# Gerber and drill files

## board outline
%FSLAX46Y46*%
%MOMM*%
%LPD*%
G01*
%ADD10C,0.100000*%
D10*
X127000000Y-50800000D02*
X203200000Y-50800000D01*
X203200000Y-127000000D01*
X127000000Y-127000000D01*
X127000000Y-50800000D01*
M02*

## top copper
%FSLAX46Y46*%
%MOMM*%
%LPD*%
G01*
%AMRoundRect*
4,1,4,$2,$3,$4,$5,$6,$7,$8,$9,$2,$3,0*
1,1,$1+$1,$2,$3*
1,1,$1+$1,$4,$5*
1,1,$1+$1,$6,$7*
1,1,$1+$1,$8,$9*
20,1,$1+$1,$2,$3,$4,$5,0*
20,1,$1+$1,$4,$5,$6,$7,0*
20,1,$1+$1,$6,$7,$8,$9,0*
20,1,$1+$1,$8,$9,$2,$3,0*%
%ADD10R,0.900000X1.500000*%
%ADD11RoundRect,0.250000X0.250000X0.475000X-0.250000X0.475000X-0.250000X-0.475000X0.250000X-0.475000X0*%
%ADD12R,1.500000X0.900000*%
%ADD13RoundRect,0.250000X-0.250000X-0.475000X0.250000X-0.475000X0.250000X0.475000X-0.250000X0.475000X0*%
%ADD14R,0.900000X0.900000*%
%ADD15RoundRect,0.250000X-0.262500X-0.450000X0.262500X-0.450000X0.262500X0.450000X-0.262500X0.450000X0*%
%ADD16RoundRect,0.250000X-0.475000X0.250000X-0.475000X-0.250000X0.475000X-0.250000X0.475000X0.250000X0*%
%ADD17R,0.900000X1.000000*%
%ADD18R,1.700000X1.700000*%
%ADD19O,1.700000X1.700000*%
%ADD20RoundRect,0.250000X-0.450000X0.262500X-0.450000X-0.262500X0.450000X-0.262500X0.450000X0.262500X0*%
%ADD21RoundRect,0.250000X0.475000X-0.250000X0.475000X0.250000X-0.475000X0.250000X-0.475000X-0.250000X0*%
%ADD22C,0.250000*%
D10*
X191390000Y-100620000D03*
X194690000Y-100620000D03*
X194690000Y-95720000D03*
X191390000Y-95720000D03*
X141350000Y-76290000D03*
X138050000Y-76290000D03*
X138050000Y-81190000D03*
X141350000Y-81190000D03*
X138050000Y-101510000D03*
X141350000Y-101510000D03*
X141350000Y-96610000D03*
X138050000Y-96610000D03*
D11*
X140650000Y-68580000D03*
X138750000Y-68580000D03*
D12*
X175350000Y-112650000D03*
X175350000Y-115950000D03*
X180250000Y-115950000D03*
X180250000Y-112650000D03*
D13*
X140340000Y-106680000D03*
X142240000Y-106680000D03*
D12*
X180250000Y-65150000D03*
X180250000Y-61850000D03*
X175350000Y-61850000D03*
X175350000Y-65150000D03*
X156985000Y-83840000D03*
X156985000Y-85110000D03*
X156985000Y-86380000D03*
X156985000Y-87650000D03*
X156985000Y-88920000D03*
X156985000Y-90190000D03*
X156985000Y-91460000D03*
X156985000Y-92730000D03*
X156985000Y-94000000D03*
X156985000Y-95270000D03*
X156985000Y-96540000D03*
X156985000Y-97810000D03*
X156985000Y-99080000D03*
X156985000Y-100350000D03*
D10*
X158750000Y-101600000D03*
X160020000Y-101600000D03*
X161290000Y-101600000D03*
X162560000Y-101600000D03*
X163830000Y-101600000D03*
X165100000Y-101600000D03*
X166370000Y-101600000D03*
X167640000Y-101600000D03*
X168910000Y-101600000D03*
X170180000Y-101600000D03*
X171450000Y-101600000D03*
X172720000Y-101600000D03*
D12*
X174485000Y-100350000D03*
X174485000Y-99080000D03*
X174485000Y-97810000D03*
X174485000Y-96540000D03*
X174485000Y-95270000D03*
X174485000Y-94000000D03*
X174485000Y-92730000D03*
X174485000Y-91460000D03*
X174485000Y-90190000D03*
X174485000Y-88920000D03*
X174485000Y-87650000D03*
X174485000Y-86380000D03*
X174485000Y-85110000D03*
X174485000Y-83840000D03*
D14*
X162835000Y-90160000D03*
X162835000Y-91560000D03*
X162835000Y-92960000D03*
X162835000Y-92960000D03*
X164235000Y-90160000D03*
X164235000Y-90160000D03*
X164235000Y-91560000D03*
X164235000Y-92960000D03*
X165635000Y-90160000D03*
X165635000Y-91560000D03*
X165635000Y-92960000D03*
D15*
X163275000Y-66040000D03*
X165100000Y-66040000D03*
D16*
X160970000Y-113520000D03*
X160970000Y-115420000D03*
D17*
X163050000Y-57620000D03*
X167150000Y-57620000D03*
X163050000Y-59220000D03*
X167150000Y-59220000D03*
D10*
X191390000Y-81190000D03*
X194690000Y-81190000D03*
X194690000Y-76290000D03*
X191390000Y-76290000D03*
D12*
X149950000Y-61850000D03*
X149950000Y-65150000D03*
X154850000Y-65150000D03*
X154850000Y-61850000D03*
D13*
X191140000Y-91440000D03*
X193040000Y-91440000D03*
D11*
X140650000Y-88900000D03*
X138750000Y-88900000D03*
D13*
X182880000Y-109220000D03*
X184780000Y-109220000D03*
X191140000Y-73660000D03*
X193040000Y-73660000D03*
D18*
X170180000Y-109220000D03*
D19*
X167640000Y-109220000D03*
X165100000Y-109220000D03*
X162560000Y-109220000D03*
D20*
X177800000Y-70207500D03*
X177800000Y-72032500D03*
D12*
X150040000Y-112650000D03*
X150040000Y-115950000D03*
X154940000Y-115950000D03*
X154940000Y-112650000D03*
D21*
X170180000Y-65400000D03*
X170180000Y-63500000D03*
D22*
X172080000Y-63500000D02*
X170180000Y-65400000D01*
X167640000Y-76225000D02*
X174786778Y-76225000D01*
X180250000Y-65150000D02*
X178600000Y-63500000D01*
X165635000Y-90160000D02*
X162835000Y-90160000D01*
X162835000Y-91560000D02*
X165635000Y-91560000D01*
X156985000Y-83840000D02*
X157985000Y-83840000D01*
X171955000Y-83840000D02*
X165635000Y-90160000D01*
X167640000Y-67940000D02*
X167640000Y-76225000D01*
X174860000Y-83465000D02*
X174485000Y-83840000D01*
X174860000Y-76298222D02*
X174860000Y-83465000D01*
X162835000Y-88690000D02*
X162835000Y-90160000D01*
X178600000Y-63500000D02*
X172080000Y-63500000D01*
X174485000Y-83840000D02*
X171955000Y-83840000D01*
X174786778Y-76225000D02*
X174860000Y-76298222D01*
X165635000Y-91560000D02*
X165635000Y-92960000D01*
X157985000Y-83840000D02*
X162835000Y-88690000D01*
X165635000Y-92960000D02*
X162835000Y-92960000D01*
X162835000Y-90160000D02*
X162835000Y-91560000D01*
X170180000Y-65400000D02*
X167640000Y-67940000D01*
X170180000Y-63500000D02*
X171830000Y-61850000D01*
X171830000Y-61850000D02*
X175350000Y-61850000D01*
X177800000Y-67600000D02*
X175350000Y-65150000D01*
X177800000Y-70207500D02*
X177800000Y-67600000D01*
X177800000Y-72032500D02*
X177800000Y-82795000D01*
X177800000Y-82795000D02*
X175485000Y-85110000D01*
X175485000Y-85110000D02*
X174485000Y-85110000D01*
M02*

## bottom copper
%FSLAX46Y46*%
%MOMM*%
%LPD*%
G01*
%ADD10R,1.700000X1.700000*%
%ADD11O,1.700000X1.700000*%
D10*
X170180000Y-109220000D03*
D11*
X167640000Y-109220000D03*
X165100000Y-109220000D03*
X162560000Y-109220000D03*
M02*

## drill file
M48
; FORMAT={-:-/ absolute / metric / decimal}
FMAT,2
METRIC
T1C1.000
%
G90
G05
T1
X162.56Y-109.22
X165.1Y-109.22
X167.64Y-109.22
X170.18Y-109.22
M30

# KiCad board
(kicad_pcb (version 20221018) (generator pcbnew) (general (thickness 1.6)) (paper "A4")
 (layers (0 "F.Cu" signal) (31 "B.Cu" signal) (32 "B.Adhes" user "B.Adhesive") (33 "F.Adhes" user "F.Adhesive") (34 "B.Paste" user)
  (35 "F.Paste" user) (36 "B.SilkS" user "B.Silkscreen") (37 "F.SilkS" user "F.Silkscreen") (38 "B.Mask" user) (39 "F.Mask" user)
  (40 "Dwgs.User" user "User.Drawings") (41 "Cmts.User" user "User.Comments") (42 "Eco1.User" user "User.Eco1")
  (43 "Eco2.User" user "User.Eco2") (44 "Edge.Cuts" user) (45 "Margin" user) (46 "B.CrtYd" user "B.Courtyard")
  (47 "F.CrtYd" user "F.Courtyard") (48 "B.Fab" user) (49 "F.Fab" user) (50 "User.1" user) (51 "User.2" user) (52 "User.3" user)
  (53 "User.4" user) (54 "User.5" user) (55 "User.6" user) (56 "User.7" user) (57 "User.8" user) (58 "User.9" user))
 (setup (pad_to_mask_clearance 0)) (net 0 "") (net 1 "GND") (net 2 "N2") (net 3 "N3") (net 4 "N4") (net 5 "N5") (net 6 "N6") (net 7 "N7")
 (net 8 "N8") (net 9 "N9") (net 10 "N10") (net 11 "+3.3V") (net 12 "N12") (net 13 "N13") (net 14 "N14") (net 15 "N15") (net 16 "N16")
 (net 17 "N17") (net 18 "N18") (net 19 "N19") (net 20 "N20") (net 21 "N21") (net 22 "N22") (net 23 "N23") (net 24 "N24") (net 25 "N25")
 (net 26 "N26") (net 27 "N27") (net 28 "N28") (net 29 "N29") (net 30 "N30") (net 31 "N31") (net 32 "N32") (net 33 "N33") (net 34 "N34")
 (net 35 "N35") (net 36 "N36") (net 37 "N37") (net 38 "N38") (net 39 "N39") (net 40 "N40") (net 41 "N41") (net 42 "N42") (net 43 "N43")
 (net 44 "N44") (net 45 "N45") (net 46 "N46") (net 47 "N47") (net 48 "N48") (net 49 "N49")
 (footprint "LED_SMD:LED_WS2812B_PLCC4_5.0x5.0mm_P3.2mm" (layer "F.Cu") (at 193.04 98.17 90)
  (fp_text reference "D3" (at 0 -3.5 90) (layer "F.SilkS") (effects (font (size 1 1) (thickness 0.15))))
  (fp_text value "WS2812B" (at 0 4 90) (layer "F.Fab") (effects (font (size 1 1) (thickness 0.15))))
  (pad "1" smd rect (at -2.45 -1.65 90) (size 1.5 0.9) (layers "F.Cu" "F.Paste" "F.Mask") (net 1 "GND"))
  (pad "2" smd rect (at -2.45 1.65 90) (size 1.5 0.9) (layers "F.Cu" "F.Paste" "F.Mask") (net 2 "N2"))
  (pad "3" smd rect (at 2.45 1.65 90) (size 1.5 0.9) (layers "F.Cu" "F.Paste" "F.Mask") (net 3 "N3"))
  (pad "4" smd rect (at 2.45 -1.65 90) (size 1.5 0.9) (layers "F.Cu" "F.Paste" "F.Mask") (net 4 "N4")))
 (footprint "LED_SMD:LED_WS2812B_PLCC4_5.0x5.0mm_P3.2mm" (layer "F.Cu") (at 139.7 78.74 -90)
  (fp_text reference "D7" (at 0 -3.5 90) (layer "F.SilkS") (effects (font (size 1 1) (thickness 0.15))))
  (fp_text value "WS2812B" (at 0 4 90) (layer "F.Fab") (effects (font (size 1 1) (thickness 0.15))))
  (pad "1" smd rect (at -2.45 -1.65 270) (size 1.5 0.9) (layers "F.Cu" "F.Paste" "F.Mask") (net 1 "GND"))
  (pad "2" smd rect (at -2.45 1.65 270) (size 1.5 0.9) (layers "F.Cu" "F.Paste" "F.Mask") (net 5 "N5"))
  (pad "3" smd rect (at 2.45 1.65 270) (size 1.5 0.9) (layers "F.Cu" "F.Paste" "F.Mask") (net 3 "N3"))
  (pad "4" smd rect (at 2.45 -1.65 270) (size 1.5 0.9) (layers "F.Cu" "F.Paste" "F.Mask") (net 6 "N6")))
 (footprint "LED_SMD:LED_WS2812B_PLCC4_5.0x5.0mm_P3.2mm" (layer "F.Cu") (at 139.7 99.06 90)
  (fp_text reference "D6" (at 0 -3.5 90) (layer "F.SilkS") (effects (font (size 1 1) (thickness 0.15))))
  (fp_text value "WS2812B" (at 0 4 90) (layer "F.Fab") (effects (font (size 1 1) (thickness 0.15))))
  (pad "1" smd rect (at -2.45 -1.65 90) (size 1.5 0.9) (layers "F.Cu" "F.Paste" "F.Mask") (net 1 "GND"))
  (pad "2" smd rect (at -2.45 1.65 90) (size 1.5 0.9) (layers "F.Cu" "F.Paste" "F.Mask") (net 6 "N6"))
  (pad "3" smd rect (at 2.45 1.65 90) (size 1.5 0.9) (layers "F.Cu" "F.Paste" "F.Mask") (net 3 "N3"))
  (pad "4" smd rect (at 2.45 -1.65 90) (size 1.5 0.9) (layers "F.Cu" "F.Paste" "F.Mask") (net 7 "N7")))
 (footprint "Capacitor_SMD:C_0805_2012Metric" (layer "F.Cu") (at 139.7 68.58 180)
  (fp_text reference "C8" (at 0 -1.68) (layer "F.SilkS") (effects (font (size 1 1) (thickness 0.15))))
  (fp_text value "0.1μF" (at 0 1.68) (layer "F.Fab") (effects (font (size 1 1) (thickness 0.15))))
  (pad "1" smd roundrect (at -0.95 0 180) (size 1 1.45) (layers "F.Cu" "F.Paste" "F.Mask") (roundrect_rratio 0.25) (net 1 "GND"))
  (pad "2" smd roundrect (at 0.95 0 180) (size 1 1.45) (layers "F.Cu" "F.Paste" "F.Mask") (roundrect_rratio 0.25) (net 3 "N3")))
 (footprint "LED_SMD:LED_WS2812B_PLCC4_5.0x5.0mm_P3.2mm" (layer "F.Cu") (at 177.8 114.3)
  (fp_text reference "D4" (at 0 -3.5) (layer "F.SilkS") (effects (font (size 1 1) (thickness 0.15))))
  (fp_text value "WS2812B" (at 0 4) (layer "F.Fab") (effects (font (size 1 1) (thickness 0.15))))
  (pad "1" smd rect (at -2.45 -1.65) (size 1.5 0.9) (layers "F.Cu" "F.Paste" "F.Mask") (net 1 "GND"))
  (pad "2" smd rect (at -2.45 1.65) (size 1.5 0.9) (layers "F.Cu" "F.Paste" "F.Mask") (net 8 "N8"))
  (pad "3" smd rect (at 2.45 1.65) (size 1.5 0.9) (layers "F.Cu" "F.Paste" "F.Mask") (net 3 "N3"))
  (pad "4" smd rect (at 2.45 -1.65) (size 1.5 0.9) (layers "F.Cu" "F.Paste" "F.Mask") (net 2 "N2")))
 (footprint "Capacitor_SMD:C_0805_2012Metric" (layer "F.Cu") (at 141.29 106.68)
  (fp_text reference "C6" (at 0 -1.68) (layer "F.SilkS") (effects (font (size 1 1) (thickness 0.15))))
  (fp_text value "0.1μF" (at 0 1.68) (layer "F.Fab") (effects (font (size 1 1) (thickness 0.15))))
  (pad "1" smd roundrect (at -0.95 0) (size 1 1.45) (layers "F.Cu" "F.Paste" "F.Mask") (roundrect_rratio 0.25) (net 1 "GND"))
  (pad "2" smd roundrect (at 0.95 0) (size 1 1.45) (layers "F.Cu" "F.Paste" "F.Mask") (roundrect_rratio 0.25) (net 3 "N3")))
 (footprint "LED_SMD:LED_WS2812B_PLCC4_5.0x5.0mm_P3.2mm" (layer "F.Cu") (at 177.8 63.5 180)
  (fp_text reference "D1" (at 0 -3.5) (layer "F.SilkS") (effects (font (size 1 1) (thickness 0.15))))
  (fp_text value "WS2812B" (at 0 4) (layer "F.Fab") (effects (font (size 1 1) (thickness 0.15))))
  (pad "1" smd rect (at -2.45 -1.65 180) (size 1.5 0.9) (layers "F.Cu" "F.Paste" "F.Mask") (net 1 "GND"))
  (pad "2" smd rect (at -2.45 1.65 180) (size 1.5 0.9) (layers "F.Cu" "F.Paste" "F.Mask") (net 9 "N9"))
  (pad "3" smd rect (at 2.45 1.65 180) (size 1.5 0.9) (layers "F.Cu" "F.Paste" "F.Mask") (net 3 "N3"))
  (pad "4" smd rect (at 2.45 -1.65 180) (size 1.5 0.9) (layers "F.Cu" "F.Paste" "F.Mask") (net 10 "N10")))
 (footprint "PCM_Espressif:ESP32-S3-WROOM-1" (layer "F.Cu") (at 165.735 92.1)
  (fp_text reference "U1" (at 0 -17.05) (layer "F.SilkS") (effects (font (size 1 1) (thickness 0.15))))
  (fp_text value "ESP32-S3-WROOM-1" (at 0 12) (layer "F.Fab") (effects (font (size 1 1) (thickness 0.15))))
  (pad "1" smd rect (at -8.75 -8.26) (size 1.5 0.9) (layers "F.Cu" "F.Paste" "F.Mask") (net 1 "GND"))
  (pad "2" smd rect (at -8.75 -6.99) (size 1.5 0.9) (layers "F.Cu" "F.Paste" "F.Mask") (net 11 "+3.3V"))
  (pad "3" smd rect (at -8.75 -5.72) (size 1.5 0.9) (layers "F.Cu" "F.Paste" "F.Mask") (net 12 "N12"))
  (pad "4" smd rect (at -8.75 -4.45) (size 1.5 0.9) (layers "F.Cu" "F.Paste" "F.Mask") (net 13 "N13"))
  (pad "5" smd rect (at -8.75 -3.18) (size 1.5 0.9) (layers "F.Cu" "F.Paste" "F.Mask") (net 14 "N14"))
  (pad "6" smd rect (at -8.75 -1.91) (size 1.5 0.9) (layers "F.Cu" "F.Paste" "F.Mask") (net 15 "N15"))
  (pad "7" smd rect (at -8.75 -0.64) (size 1.5 0.9) (layers "F.Cu" "F.Paste" "F.Mask") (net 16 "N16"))
  (pad "8" smd rect (at -8.75 0.63) (size 1.5 0.9) (layers "F.Cu" "F.Paste" "F.Mask") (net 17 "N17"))
  (pad "9" smd rect (at -8.75 1.9) (size 1.5 0.9) (layers "F.Cu" "F.Paste" "F.Mask") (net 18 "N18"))
  (pad "10" smd rect (at -8.75 3.17) (size 1.5 0.9) (layers "F.Cu" "F.Paste" "F.Mask") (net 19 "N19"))
  (pad "11" smd rect (at -8.75 4.44) (size 1.5 0.9) (layers "F.Cu" "F.Paste" "F.Mask") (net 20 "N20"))
  (pad "12" smd rect (at -8.75 5.71) (size 1.5 0.9) (layers "F.Cu" "F.Paste" "F.Mask") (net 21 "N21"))
  (pad "13" smd rect (at -8.75 6.98) (size 1.5 0.9) (layers "F.Cu" "F.Paste" "F.Mask") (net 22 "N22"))
  (pad "14" smd rect (at -8.75 8.25) (size 1.5 0.9) (layers "F.Cu" "F.Paste" "F.Mask") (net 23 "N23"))
  (pad "15" smd rect (at -6.985 9.5 90) (size 1.5 0.9) (layers "F.Cu" "F.Paste" "F.Mask") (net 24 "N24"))
  (pad "16" smd rect (at -5.715 9.5 90) (size 1.5 0.9) (layers "F.Cu" "F.Paste" "F.Mask") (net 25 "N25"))
  (pad "17" smd rect (at -4.445 9.5 90) (size 1.5 0.9) (layers "F.Cu" "F.Paste" "F.Mask") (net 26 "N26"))
  (pad "18" smd rect (at -3.175 9.5 90) (size 1.5 0.9) (layers "F.Cu" "F.Paste" "F.Mask") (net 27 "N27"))
  (pad "19" smd rect (at -1.905 9.5 90) (size 1.5 0.9) (layers "F.Cu" "F.Paste" "F.Mask") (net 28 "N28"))
  (pad "20" smd rect (at -0.635 9.5 90) (size 1.5 0.9) (layers "F.Cu" "F.Paste" "F.Mask") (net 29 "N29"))
  (pad "21" smd rect (at 0.635 9.5 90) (size 1.5 0.9) (layers "F.Cu" "F.Paste" "F.Mask") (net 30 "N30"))
  (pad "22" smd rect (at 1.905 9.5 90) (size 1.5 0.9) (layers "F.Cu" "F.Paste" "F.Mask") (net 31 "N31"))
  (pad "23" smd rect (at 3.175 9.5 90) (size 1.5 0.9) (layers "F.Cu" "F.Paste" "F.Mask") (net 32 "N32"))
  (pad "24" smd rect (at 4.445 9.5 90) (size 1.5 0.9) (layers "F.Cu" "F.Paste" "F.Mask") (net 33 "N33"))
  (pad "25" smd rect (at 5.715 9.5 90) (size 1.5 0.9) (layers "F.Cu" "F.Paste" "F.Mask") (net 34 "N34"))
  (pad "26" smd rect (at 6.985 9.5 90) (size 1.5 0.9) (layers "F.Cu" "F.Paste" "F.Mask") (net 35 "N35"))
  (pad "27" smd rect (at 8.75 8.25 180) (size 1.5 0.9) (layers "F.Cu" "F.Paste" "F.Mask") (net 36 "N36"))
  (pad "28" smd rect (at 8.75 6.98 180) (size 1.5 0.9) (layers "F.Cu" "F.Paste" "F.Mask") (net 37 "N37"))
  (pad "29" smd rect (at 8.75 5.71 180) (size 1.5 0.9) (layers "F.Cu" "F.Paste" "F.Mask") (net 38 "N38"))
  (pad "30" smd rect (at 8.75 4.44 180) (size 1.5 0.9) (layers "F.Cu" "F.Paste" "F.Mask") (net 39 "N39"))
  (pad "31" smd rect (at 8.75 3.17 180) (size 1.5 0.9) (layers "F.Cu" "F.Paste" "F.Mask") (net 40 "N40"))
  (pad "32" smd rect (at 8.75 1.9 180) (size 1.5 0.9) (layers "F.Cu" "F.Paste" "F.Mask") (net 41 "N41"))
  (pad "33" smd rect (at 8.75 0.63 180) (size 1.5 0.9) (layers "F.Cu" "F.Paste" "F.Mask") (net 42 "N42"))
  (pad "34" smd rect (at 8.75 -0.64 180) (size 1.5 0.9) (layers "F.Cu" "F.Paste" "F.Mask") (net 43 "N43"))
  (pad "35" smd rect (at 8.75 -1.91 180) (size 1.5 0.9) (layers "F.Cu" "F.Paste" "F.Mask") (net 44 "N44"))
  (pad "36" smd rect (at 8.75 -3.18 180) (size 1.5 0.9) (layers "F.Cu" "F.Paste" "F.Mask") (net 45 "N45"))
  (pad "37" smd rect (at 8.75 -4.45 180) (size 1.5 0.9) (layers "F.Cu" "F.Paste" "F.Mask") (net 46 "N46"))
  (pad "38" smd rect (at 8.75 -5.72 180) (size 1.5 0.9) (layers "F.Cu" "F.Paste" "F.Mask") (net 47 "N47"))
  (pad "39" smd rect (at 8.75 -6.99 180) (size 1.5 0.9) (layers "F.Cu" "F.Paste" "F.Mask") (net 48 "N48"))
  (pad "40" smd rect (at 8.75 -8.26 180) (size 1.5 0.9) (layers "F.Cu" "F.Paste" "F.Mask") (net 1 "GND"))
  (pad "41" smd rect (at -2.9 -1.94 180) (size 0.9 0.9) (layers "F.Cu" "F.Paste" "F.Mask") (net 1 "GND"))
  (pad "41" smd rect (at -2.9 -0.54 180) (size 0.9 0.9) (layers "F.Cu" "F.Paste" "F.Mask") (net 1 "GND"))
  (pad "41" smd rect (at -2.9 0.86 180) (size 0.9 0.9) (layers "F.Cu" "F.Paste" "F.Mask") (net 1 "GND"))
  (pad "41" smd rect (at -2.9 0.86 180) (size 0.9 0.9) (layers "F.Cu" "F.Paste" "F.Mask") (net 1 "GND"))
  (pad "41" smd rect (at -1.5 -1.94 180) (size 0.9 0.9) (layers "F.Cu" "F.Paste" "F.Mask") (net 1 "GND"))
  (pad "41" smd rect (at -1.5 -1.94 180) (size 0.9 0.9) (layers "F.Cu" "F.Paste" "F.Mask") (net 1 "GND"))
  (pad "41" smd rect (at -1.5 -0.54 180) (size 0.9 0.9) (layers "F.Cu" "F.Paste" "F.Mask") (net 1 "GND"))
  (pad "41" smd rect (at -1.5 0.86 180) (size 0.9 0.9) (layers "F.Cu" "F.Paste" "F.Mask") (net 1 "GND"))
  (pad "41" smd rect (at -0.1 -1.94 180) (size 0.9 0.9) (layers "F.Cu" "F.Paste" "F.Mask") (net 1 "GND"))
  (pad "41" smd rect (at -0.1 -0.54 180) (size 0.9 0.9) (layers "F.Cu" "F.Paste" "F.Mask") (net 1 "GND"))
  (pad "41" smd rect (at -0.1 0.86 180) (size 0.9 0.9) (layers "F.Cu" "F.Paste" "F.Mask") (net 1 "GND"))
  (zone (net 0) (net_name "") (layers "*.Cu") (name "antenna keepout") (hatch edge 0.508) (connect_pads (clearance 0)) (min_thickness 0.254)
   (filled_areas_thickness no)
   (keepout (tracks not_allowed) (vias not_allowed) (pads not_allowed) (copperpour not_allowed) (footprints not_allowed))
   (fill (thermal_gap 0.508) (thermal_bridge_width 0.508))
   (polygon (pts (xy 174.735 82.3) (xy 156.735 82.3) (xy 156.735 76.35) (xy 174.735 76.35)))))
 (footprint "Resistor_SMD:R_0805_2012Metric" (layer "F.Cu") (at 164.1875 66.04)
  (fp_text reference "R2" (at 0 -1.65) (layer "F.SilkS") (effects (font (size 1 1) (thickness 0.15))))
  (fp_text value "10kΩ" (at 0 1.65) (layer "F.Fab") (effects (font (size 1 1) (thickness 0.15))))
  (pad "1" smd roundrect (at -0.9125 0) (size 1.025 1.4) (layers "F.Cu" "F.Paste" "F.Mask") (roundrect_rratio 0.243902) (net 13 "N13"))
  (pad "2" smd roundrect (at 0.9125 0) (size 1.025 1.4) (layers "F.Cu" "F.Paste" "F.Mask") (roundrect_rratio 0.243902) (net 1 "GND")))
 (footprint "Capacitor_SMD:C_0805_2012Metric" (layer "F.Cu") (at 160.97 114.47 -90)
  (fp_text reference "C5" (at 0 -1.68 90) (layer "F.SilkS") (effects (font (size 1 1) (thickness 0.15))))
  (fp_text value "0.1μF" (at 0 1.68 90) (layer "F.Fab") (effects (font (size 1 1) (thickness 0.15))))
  (pad "1" smd roundrect (at -0.95 0 270) (size 1 1.45) (layers "F.Cu" "F.Paste" "F.Mask") (roundrect_rratio 0.25) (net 1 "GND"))
  (pad "2" smd roundrect (at 0.95 0 270) (size 1 1.45) (layers "F.Cu" "F.Paste" "F.Mask") (roundrect_rratio 0.25) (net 3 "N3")))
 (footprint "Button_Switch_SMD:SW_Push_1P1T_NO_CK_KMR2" (layer "F.Cu") (at 165.1 58.42)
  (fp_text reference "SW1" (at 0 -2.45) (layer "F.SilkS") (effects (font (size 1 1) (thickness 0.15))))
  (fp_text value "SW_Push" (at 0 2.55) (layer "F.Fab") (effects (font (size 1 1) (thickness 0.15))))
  (pad "1" smd rect (at -2.05 -0.8) (size 0.9 1) (layers "F.Cu" "F.Paste" "F.Mask") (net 3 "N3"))
  (pad "1" smd rect (at 2.05 -0.8) (size 0.9 1) (layers "F.Cu" "F.Paste" "F.Mask") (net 3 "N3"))
  (pad "2" smd rect (at -2.05 0.8) (size 0.9 1) (layers "F.Cu" "F.Paste" "F.Mask") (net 13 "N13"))
  (pad "2" smd rect (at 2.05 0.8) (size 0.9 1) (layers "F.Cu" "F.Paste" "F.Mask") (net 13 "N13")))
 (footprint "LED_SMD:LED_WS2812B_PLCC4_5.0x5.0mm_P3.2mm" (layer "F.Cu") (at 193.04 78.74 90)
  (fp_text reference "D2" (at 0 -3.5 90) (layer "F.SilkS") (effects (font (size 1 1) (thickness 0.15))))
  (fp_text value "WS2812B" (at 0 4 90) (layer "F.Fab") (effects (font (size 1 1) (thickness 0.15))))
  (pad "1" smd rect (at -2.45 -1.65 90) (size 1.5 0.9) (layers "F.Cu" "F.Paste" "F.Mask") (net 1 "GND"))
  (pad "2" smd rect (at -2.45 1.65 90) (size 1.5 0.9) (layers "F.Cu" "F.Paste" "F.Mask") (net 4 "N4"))
  (pad "3" smd rect (at 2.45 1.65 90) (size 1.5 0.9) (layers "F.Cu" "F.Paste" "F.Mask") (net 3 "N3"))
  (pad "4" smd rect (at 2.45 -1.65 90) (size 1.5 0.9) (layers "F.Cu" "F.Paste" "F.Mask") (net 9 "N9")))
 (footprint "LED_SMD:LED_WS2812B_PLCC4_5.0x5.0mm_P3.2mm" (layer "F.Cu") (at 152.4 63.5)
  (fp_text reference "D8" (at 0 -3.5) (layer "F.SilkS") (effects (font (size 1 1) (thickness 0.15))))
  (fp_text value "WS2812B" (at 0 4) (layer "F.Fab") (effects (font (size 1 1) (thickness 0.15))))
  (pad "1" smd rect (at -2.45 -1.65) (size 1.5 0.9) (layers "F.Cu" "F.Paste" "F.Mask") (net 1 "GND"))
  (pad "2" smd rect (at -2.45 1.65) (size 1.5 0.9) (layers "F.Cu" "F.Paste" "F.Mask") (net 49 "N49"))
  (pad "3" smd rect (at 2.45 1.65) (size 1.5 0.9) (layers "F.Cu" "F.Paste" "F.Mask") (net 3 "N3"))
  (pad "4" smd rect (at 2.45 -1.65) (size 1.5 0.9) (layers "F.Cu" "F.Paste" "F.Mask") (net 5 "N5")))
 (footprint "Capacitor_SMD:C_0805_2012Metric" (layer "F.Cu") (at 192.09 91.44)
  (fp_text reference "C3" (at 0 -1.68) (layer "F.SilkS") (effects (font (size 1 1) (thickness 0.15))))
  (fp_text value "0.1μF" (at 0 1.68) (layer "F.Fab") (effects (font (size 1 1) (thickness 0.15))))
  (pad "1" smd roundrect (at -0.95 0) (size 1 1.45) (layers "F.Cu" "F.Paste" "F.Mask") (roundrect_rratio 0.25) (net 1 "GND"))
  (pad "2" smd roundrect (at 0.95 0) (size 1 1.45) (layers "F.Cu" "F.Paste" "F.Mask") (roundrect_rratio 0.25) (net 3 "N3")))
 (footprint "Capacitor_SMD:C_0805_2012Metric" (layer "F.Cu") (at 139.7 88.9 180)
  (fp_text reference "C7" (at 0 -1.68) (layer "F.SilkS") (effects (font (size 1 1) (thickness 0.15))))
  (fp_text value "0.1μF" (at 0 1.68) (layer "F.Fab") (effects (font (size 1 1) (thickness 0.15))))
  (pad "1" smd roundrect (at -0.95 0 180) (size 1 1.45) (layers "F.Cu" "F.Paste" "F.Mask") (roundrect_rratio 0.25) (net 1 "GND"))
  (pad "2" smd roundrect (at 0.95 0 180) (size 1 1.45) (layers "F.Cu" "F.Paste" "F.Mask") (roundrect_rratio 0.25) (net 3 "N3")))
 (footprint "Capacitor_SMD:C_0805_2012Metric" (layer "F.Cu") (at 183.83 109.22)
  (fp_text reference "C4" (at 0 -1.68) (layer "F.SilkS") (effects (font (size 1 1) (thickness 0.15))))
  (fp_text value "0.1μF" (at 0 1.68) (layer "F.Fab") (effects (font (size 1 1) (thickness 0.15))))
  (pad "1" smd roundrect (at -0.95 0) (size 1 1.45) (layers "F.Cu" "F.Paste" "F.Mask") (roundrect_rratio 0.25) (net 1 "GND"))
  (pad "2" smd roundrect (at 0.95 0) (size 1 1.45) (layers "F.Cu" "F.Paste" "F.Mask") (roundrect_rratio 0.25) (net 3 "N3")))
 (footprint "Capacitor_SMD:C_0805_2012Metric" (layer "F.Cu") (at 192.09 73.66)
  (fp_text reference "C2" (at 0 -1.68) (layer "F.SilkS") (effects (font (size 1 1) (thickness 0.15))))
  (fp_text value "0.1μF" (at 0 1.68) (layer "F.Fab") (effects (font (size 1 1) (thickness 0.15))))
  (pad "1" smd roundrect (at -0.95 0) (size 1 1.45) (layers "F.Cu" "F.Paste" "F.Mask") (roundrect_rratio 0.25) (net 1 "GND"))
  (pad "2" smd roundrect (at 0.95 0) (size 1 1.45) (layers "F.Cu" "F.Paste" "F.Mask") (roundrect_rratio 0.25) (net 3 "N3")))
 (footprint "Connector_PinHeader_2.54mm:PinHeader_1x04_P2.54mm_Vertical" (layer "F.Cu") (at 170.18 109.22 -90)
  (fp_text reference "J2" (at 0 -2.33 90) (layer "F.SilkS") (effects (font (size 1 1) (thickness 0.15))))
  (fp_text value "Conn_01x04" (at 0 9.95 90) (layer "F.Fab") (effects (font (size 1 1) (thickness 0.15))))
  (pad "1" thru_hole rect (at 0 0 270) (size 1.7 1.7) (drill 1) (layers "*.Cu" "*.Mask") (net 1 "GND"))
  (pad "2" thru_hole oval (at 0 2.54 270) (size 1.7 1.7) (drill 1) (layers "*.Cu" "*.Mask") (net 3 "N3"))
  (pad "3" thru_hole oval (at 0 5.08 270) (size 1.7 1.7) (drill 1) (layers "*.Cu" "*.Mask") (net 47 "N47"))
  (pad "4" thru_hole oval (at 0 7.62 270) (size 1.7 1.7) (drill 1) (layers "*.Cu" "*.Mask") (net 24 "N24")))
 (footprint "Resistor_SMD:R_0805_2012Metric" (layer "F.Cu") (at 177.8 71.12 -90)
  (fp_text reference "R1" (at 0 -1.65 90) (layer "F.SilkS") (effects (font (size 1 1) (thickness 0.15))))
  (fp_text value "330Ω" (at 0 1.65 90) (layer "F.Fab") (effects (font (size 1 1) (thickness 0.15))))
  (pad "1" smd roundrect (at -0.9125 0 270) (size 1.025 1.4) (layers "F.Cu" "F.Paste" "F.Mask") (roundrect_rratio 0.243902) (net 10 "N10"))
  (pad "2" smd roundrect (at 0.9125 0 270) (size 1.025 1.4) (layers "F.Cu" "F.Paste" "F.Mask") (roundrect_rratio 0.243902) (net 48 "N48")))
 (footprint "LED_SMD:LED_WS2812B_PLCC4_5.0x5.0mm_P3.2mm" (layer "F.Cu") (at 152.49 114.3)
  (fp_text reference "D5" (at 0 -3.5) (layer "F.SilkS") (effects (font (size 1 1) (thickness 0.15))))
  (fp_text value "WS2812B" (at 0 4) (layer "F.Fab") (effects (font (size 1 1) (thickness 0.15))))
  (pad "1" smd rect (at -2.45 -1.65) (size 1.5 0.9) (layers "F.Cu" "F.Paste" "F.Mask") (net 1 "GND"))
  (pad "2" smd rect (at -2.45 1.65) (size 1.5 0.9) (layers "F.Cu" "F.Paste" "F.Mask") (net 7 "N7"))
  (pad "3" smd rect (at 2.45 1.65) (size 1.5 0.9) (layers "F.Cu" "F.Paste" "F.Mask") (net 3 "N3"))
  (pad "4" smd rect (at 2.45 -1.65) (size 1.5 0.9) (layers "F.Cu" "F.Paste" "F.Mask") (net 8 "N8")))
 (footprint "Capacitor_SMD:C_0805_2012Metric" (layer "F.Cu") (at 170.18 64.45 90)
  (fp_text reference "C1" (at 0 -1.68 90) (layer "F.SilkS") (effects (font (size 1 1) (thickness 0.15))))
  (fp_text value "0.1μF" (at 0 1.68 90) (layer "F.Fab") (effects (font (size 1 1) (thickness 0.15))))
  (pad "1" smd roundrect (at -0.95 0 90) (size 1 1.45) (layers "F.Cu" "F.Paste" "F.Mask") (roundrect_rratio 0.25) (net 1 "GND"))
  (pad "2" smd roundrect (at 0.95 0 90) (size 1 1.45) (layers "F.Cu" "F.Paste" "F.Mask") (roundrect_rratio 0.25) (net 3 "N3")))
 (gr_rect (start 127 50.8) (end 203.2 127) (stroke (width 0.1) (type default)) (fill none) (layer "Edge.Cuts"))
 (segment (start 172.08 63.5) (end 170.18 65.4) (width 0.25) (layer "F.Cu") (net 1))
 (segment (start 167.64 76.225) (end 174.786778 76.225) (width 0.25) (layer "F.Cu") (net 1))
 (segment (start 180.25 65.15) (end 178.6 63.5) (width 0.25) (layer "F.Cu") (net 1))
 (segment (start 165.635 90.16) (end 162.835 90.16) (width 0.25) (layer "F.Cu") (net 1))
 (segment (start 162.835 91.56) (end 165.635 91.56) (width 0.25) (layer "F.Cu") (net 1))
 (segment (start 156.985 83.84) (end 157.985 83.84) (width 0.25) (layer "F.Cu") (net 1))
 (segment (start 171.955 83.84) (end 165.635 90.16) (width 0.25) (layer "F.Cu") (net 1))
 (segment (start 167.64 67.94) (end 167.64 76.225) (width 0.25) (layer "F.Cu") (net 1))
 (segment (start 174.86 83.465) (end 174.485 83.84) (width 0.25) (layer "F.Cu") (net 1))
 (segment (start 174.86 76.298222) (end 174.86 83.465) (width 0.25) (layer "F.Cu") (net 1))
 (segment (start 162.835 88.69) (end 162.835 90.16) (width 0.25) (layer "F.Cu") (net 1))
 (segment (start 178.6 63.5) (end 172.08 63.5) (width 0.25) (layer "F.Cu") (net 1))
 (segment (start 174.485 83.84) (end 171.955 83.84) (width 0.25) (layer "F.Cu") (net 1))
 (segment (start 174.786778 76.225) (end 174.86 76.298222) (width 0.25) (layer "F.Cu") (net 1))
 (segment (start 165.635 91.56) (end 165.635 92.96) (width 0.25) (layer "F.Cu") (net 1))
 (segment (start 157.985 83.84) (end 162.835 88.69) (width 0.25) (layer "F.Cu") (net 1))
 (segment (start 165.635 92.96) (end 162.835 92.96) (width 0.25) (layer "F.Cu") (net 1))
 (segment (start 162.835 90.16) (end 162.835 91.56) (width 0.25) (layer "F.Cu") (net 1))
 (segment (start 170.18 65.4) (end 167.64 67.94) (width 0.25) (layer "F.Cu") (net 1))
 (segment (start 170.18 63.5) (end 171.83 61.85) (width 0.25) (layer "F.Cu") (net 3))
 (segment (start 171.83 61.85) (end 175.35 61.85) (width 0.25) (layer "F.Cu") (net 3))
 (segment (start 177.8 67.6) (end 175.35 65.15) (width 0.25) (layer "F.Cu") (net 10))
 (segment (start 177.8 70.2075) (end 177.8 67.6) (width 0.25) (layer "F.Cu") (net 10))
 (segment (start 177.8 72.0325) (end 177.8 82.795) (width 0.25) (layer "F.Cu") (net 48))
 (segment (start 177.8 82.795) (end 175.485 85.11) (width 0.25) (layer "F.Cu") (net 48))
 (segment (start 175.485 85.11) (end 174.485 85.11) (width 0.25) (layer "F.Cu") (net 48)))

